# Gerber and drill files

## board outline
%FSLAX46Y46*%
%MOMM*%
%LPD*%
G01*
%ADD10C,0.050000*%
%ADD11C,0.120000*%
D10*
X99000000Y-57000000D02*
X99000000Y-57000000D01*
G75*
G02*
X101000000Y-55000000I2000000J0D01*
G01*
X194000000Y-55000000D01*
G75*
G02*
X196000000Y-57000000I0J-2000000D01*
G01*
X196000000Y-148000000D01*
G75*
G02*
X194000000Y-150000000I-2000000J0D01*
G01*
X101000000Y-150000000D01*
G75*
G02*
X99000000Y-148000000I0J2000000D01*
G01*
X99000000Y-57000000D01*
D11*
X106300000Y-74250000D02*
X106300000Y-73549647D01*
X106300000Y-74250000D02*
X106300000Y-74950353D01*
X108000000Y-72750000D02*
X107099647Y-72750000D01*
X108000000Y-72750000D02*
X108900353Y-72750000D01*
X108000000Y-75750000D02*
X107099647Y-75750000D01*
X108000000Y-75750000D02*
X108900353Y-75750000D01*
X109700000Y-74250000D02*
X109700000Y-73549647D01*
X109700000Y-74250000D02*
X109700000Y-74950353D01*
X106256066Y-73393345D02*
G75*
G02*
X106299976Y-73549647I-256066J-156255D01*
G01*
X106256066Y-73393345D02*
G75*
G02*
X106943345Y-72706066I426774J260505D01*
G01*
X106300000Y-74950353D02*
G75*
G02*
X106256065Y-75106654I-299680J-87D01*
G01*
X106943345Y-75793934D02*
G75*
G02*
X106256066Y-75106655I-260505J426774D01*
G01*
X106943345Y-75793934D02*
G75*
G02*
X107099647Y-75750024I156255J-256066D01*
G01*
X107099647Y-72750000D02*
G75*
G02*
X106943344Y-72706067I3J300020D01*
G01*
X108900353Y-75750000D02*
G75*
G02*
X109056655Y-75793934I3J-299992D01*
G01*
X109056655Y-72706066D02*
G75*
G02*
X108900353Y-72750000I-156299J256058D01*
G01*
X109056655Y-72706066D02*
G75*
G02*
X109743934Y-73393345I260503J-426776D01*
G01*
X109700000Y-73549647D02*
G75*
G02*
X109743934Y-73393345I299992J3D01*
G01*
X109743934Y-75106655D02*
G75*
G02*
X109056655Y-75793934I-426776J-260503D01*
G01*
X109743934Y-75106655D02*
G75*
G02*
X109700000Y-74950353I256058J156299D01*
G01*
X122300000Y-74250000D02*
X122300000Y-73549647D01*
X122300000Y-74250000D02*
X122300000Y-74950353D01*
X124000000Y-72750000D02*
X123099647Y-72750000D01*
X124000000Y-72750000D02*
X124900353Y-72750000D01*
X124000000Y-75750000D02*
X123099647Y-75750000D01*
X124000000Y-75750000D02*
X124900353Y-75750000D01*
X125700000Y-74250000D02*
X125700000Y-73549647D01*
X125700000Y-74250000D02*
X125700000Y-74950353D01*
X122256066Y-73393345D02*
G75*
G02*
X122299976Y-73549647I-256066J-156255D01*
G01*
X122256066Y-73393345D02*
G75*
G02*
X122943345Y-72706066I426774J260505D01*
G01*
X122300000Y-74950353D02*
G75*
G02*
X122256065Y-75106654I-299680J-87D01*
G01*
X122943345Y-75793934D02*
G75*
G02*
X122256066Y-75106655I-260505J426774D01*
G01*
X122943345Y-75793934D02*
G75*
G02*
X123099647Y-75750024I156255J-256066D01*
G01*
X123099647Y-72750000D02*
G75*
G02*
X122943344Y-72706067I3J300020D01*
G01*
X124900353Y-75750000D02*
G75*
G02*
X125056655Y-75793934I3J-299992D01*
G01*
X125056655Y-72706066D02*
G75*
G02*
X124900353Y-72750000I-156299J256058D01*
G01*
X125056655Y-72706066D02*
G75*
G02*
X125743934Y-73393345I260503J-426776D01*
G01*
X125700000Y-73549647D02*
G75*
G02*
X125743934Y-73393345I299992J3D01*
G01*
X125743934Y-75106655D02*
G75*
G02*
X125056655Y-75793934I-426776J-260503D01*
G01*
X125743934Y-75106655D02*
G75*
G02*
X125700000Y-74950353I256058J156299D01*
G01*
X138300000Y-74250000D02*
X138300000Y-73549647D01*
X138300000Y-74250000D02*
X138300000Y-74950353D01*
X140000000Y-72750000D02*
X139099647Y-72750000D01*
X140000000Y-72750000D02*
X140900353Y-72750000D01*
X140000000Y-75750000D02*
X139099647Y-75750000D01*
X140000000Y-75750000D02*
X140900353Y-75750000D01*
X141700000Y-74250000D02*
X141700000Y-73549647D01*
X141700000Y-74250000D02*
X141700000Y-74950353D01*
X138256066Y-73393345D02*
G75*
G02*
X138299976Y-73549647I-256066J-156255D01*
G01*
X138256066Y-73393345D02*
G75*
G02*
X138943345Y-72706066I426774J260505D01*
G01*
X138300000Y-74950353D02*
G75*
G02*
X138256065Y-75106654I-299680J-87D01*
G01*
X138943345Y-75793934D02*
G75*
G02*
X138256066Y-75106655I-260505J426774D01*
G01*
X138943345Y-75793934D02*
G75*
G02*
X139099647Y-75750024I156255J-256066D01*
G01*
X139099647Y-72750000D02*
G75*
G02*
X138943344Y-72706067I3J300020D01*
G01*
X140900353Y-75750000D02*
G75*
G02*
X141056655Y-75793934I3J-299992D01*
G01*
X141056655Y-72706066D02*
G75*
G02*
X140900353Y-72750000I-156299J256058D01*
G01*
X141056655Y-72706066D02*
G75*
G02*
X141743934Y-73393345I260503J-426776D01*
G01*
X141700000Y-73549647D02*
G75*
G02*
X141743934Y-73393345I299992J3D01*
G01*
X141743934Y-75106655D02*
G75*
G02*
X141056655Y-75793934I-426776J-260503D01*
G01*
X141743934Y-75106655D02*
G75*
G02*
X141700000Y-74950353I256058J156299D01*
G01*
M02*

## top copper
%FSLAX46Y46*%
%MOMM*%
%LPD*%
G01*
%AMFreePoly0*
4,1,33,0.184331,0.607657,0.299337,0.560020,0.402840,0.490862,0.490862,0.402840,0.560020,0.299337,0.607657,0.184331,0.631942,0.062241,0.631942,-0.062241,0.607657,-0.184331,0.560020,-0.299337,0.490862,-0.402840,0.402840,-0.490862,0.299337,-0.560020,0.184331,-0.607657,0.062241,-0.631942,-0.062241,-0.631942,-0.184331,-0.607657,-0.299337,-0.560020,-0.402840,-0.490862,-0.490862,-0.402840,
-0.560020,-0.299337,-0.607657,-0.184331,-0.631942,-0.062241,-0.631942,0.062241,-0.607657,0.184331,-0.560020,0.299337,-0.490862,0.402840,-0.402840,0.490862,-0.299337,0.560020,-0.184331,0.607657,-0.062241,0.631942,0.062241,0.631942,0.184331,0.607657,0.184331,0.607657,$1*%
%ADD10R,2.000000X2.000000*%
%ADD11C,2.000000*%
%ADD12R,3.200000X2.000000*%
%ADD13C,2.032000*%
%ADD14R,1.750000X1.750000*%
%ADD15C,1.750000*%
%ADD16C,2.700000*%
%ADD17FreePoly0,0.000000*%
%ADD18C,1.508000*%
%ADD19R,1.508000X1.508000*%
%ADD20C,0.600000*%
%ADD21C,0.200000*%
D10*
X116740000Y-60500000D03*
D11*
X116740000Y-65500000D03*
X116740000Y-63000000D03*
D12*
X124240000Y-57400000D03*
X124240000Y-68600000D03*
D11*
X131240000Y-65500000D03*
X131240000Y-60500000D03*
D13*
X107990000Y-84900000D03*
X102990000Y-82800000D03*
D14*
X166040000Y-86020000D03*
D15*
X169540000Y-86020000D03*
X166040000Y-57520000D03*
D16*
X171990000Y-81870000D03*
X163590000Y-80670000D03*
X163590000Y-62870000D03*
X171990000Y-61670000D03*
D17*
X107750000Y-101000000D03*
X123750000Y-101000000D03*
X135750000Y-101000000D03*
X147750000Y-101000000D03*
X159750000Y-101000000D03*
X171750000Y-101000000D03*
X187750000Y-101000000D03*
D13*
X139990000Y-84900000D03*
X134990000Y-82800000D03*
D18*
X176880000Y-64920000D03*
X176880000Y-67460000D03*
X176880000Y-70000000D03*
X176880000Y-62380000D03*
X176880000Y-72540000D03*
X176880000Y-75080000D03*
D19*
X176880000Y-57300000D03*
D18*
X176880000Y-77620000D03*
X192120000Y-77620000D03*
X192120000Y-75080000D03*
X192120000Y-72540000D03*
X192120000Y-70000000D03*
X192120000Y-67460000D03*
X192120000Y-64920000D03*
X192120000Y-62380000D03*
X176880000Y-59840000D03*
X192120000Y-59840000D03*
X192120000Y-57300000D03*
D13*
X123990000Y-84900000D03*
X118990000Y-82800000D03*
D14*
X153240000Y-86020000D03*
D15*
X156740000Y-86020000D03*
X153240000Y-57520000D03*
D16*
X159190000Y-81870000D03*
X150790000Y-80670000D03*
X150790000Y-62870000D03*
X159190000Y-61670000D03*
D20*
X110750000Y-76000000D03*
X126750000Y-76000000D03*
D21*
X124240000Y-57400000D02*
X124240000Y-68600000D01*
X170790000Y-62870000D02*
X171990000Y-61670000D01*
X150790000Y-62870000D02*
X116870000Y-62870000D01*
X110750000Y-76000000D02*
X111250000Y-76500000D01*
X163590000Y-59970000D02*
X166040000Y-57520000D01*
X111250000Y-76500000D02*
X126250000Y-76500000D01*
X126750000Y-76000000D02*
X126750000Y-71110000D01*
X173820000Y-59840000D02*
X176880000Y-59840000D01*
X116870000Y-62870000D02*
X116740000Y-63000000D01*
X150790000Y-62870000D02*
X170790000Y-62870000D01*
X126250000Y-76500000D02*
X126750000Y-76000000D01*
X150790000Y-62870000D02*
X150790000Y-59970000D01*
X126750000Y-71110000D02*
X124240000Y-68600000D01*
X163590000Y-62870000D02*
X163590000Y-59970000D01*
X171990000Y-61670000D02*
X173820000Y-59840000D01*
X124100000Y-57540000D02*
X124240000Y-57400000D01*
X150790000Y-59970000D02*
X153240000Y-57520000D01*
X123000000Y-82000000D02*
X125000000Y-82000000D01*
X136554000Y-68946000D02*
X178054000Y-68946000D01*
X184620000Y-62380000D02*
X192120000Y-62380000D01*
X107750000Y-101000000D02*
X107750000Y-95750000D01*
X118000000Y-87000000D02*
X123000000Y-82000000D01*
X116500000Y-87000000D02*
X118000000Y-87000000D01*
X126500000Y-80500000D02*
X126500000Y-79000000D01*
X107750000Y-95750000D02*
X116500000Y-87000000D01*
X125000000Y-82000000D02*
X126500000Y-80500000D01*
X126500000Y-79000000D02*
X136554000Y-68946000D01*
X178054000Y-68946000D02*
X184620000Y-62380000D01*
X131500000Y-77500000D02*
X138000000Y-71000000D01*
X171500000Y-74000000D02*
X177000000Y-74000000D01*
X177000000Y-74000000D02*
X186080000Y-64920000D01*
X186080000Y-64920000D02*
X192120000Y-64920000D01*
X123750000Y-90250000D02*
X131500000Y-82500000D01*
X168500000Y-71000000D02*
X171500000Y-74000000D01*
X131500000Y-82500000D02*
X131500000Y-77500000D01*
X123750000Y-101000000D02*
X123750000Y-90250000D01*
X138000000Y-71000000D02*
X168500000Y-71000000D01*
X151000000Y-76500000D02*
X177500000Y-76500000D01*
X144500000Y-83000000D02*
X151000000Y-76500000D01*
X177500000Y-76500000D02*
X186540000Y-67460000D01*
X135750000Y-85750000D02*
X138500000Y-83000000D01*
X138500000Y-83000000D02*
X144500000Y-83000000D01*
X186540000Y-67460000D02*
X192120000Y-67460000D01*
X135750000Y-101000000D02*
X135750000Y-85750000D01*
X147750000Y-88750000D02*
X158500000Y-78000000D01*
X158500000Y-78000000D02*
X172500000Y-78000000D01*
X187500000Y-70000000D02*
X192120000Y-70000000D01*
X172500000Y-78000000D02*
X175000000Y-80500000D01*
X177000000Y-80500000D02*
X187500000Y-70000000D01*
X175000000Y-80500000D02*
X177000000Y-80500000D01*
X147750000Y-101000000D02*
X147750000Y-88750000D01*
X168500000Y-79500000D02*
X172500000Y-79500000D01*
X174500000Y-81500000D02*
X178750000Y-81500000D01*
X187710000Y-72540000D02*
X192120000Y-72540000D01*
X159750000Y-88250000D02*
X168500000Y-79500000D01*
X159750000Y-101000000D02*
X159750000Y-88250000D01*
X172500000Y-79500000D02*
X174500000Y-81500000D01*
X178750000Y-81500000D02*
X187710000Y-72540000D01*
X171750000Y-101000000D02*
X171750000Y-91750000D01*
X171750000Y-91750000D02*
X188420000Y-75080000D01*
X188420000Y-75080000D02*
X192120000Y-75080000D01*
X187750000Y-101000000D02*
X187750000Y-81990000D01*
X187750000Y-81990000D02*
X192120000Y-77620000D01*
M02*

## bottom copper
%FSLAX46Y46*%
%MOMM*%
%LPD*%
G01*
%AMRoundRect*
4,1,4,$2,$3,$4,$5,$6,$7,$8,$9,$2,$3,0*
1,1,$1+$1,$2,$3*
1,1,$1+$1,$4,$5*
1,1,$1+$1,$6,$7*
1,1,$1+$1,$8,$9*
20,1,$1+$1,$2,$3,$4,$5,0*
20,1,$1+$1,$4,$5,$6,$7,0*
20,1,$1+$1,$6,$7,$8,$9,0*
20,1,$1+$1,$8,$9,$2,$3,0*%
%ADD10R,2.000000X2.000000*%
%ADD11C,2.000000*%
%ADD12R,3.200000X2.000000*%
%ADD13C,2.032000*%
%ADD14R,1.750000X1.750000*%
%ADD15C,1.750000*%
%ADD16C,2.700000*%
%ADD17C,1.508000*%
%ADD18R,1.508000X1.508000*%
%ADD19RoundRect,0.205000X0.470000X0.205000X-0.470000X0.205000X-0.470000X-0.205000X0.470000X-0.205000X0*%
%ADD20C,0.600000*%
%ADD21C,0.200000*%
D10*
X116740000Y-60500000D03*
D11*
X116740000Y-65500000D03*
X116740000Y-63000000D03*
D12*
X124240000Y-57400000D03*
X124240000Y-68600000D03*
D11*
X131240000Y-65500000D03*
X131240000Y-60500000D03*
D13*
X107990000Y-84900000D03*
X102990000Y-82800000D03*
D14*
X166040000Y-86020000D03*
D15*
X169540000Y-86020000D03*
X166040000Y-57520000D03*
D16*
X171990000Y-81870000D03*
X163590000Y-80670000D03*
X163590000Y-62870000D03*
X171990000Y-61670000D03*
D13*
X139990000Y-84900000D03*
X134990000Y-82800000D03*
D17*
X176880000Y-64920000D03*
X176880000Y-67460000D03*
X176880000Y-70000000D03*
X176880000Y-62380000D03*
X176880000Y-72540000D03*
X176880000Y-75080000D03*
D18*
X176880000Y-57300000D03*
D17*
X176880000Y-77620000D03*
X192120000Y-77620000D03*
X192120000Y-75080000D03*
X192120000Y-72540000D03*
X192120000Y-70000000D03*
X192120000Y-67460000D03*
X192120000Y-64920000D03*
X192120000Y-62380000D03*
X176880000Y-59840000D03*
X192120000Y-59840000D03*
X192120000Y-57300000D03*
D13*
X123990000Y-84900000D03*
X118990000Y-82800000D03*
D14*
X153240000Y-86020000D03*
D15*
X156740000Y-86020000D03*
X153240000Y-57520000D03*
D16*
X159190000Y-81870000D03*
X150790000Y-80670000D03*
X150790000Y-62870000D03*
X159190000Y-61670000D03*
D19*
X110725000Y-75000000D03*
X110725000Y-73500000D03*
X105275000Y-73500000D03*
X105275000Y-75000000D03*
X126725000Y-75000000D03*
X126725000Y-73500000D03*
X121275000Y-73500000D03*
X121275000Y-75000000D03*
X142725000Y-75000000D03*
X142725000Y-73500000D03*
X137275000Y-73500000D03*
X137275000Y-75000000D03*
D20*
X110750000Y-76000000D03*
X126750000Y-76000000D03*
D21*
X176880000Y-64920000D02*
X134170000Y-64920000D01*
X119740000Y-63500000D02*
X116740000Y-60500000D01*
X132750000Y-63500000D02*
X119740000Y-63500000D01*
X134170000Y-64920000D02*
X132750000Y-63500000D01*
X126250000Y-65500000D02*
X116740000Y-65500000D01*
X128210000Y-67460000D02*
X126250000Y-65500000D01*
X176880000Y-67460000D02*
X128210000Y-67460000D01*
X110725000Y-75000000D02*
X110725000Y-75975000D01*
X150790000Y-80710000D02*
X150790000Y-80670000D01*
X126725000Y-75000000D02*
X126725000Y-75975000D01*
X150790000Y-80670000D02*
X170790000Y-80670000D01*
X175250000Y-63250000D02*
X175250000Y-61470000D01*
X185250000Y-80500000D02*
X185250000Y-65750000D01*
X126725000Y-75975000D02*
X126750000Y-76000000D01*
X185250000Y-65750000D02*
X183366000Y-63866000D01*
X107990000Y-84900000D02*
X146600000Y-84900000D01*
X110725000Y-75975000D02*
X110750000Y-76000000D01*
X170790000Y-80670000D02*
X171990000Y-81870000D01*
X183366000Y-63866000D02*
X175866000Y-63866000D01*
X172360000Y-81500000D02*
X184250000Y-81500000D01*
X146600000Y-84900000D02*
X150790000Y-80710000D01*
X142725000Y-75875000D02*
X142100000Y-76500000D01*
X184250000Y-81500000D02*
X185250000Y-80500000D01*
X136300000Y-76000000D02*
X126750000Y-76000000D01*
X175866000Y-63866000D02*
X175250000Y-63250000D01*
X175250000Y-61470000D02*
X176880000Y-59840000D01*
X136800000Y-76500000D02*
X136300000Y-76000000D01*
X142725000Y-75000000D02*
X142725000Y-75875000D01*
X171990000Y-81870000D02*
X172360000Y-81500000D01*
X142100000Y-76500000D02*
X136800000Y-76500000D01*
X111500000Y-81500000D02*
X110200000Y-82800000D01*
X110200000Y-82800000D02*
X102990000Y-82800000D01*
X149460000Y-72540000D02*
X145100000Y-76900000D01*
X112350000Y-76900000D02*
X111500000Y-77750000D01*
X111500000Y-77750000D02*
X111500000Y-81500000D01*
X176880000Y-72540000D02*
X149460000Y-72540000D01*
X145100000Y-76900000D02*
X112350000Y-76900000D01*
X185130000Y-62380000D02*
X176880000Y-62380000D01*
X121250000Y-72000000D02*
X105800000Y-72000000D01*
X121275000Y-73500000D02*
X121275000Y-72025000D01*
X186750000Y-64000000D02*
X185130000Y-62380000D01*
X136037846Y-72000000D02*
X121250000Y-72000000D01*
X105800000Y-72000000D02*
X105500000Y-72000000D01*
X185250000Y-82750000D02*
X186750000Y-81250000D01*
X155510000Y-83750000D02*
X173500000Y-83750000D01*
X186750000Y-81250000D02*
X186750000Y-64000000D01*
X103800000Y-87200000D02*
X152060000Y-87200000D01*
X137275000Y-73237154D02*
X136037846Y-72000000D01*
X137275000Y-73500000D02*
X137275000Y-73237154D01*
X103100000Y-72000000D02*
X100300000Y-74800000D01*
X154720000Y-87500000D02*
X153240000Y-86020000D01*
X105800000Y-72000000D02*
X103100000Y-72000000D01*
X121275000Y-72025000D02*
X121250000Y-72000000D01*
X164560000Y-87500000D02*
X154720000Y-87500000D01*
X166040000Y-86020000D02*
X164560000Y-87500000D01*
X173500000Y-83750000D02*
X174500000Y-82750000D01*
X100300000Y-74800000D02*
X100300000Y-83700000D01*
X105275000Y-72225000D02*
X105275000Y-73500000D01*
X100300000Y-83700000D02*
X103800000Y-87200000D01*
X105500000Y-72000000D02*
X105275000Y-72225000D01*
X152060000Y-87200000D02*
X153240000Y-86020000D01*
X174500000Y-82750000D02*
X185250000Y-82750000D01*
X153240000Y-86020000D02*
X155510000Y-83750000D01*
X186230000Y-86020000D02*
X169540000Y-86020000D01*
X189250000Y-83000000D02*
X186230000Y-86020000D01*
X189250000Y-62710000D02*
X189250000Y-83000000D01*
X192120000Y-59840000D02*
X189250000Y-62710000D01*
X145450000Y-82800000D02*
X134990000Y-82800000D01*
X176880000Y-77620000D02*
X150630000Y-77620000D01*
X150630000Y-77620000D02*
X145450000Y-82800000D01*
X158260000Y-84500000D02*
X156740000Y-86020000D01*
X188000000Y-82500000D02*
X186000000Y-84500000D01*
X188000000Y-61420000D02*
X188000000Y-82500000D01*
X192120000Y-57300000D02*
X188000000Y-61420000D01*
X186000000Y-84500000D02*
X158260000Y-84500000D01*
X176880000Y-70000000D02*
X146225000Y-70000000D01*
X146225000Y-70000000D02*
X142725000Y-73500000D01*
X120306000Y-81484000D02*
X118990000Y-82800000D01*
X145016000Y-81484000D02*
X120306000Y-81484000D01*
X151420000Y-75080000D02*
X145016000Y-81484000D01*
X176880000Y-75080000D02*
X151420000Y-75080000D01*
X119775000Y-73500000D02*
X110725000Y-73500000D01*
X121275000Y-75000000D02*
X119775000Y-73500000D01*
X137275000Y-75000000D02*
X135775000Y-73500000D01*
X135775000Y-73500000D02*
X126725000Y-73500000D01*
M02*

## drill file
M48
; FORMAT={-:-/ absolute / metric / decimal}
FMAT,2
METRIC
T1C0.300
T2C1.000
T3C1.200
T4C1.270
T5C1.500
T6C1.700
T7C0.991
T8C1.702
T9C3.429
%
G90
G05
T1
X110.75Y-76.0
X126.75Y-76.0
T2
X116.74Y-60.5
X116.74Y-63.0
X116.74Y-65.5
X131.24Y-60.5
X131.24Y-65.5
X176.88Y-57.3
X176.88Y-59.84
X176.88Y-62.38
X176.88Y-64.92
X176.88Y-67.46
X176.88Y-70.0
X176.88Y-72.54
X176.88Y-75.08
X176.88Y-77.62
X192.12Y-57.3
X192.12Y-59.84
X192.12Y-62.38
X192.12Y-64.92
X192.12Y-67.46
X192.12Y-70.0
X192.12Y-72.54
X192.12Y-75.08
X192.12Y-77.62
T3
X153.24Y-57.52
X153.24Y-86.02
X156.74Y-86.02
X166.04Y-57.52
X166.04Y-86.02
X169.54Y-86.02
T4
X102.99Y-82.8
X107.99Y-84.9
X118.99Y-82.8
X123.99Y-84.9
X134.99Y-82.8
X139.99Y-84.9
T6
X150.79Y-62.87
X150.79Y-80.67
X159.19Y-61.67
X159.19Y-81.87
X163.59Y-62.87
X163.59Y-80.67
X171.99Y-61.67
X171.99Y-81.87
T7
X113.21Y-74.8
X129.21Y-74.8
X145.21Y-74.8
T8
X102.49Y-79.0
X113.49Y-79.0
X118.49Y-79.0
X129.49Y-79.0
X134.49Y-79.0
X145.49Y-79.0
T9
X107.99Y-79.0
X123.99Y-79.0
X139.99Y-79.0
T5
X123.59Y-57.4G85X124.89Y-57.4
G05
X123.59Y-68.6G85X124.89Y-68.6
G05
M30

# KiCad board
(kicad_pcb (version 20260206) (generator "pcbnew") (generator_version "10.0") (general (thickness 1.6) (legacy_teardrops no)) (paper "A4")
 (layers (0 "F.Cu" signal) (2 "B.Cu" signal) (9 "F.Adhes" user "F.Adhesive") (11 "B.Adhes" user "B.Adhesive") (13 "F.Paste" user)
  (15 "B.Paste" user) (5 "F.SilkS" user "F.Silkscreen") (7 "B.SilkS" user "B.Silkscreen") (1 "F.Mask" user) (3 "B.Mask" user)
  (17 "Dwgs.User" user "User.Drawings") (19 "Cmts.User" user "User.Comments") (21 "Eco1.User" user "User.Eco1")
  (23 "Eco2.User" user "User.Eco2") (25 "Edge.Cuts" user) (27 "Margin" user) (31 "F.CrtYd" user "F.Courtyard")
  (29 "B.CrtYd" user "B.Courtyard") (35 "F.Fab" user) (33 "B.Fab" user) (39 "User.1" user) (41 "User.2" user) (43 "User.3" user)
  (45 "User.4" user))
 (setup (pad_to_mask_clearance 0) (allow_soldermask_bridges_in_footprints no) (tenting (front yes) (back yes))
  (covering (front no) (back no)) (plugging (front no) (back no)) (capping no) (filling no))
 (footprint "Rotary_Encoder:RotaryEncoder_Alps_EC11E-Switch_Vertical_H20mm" (layer "F.Cu") (at 116.74 60.5)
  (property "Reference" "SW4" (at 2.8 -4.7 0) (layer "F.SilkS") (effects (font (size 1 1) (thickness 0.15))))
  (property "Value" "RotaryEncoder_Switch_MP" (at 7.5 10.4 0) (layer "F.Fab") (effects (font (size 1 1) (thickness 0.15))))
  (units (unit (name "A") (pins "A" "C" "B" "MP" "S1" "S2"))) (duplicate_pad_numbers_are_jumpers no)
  (pad "A" thru_hole rect (at 0 0) (size 2 2) (drill 1) (layers "*.Cu" "*.Mask") (remove_unused_layers no) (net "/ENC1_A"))
  (pad "B" thru_hole circle (at 0 5) (size 2 2) (drill 1) (layers "*.Cu" "*.Mask") (remove_unused_layers no) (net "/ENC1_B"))
  (pad "C" thru_hole circle (at 0 2.5) (size 2 2) (drill 1) (layers "*.Cu" "*.Mask") (remove_unused_layers no) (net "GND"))
  (pad "MP" thru_hole rect (at 7.5 -3.1) (size 3.2 2) (drill oval 2.8 1.5) (layers "*.Cu" "*.Mask") (remove_unused_layers no) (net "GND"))
  (pad "MP" thru_hole rect (at 7.5 8.1) (size 3.2 2) (drill oval 2.8 1.5) (layers "*.Cu" "*.Mask") (remove_unused_layers no) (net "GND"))
  (pad "S1" thru_hole circle (at 14.5 5) (size 2 2) (drill 1) (layers "*.Cu" "*.Mask") (remove_unused_layers no)
   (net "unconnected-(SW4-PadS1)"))
  (pad "S2" thru_hole circle (at 14.5 0) (size 2 2) (drill 1) (layers "*.Cu" "*.Mask") (remove_unused_layers no)
   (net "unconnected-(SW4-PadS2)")))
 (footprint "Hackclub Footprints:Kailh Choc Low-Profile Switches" (layer "F.Cu") (at 107.99 79)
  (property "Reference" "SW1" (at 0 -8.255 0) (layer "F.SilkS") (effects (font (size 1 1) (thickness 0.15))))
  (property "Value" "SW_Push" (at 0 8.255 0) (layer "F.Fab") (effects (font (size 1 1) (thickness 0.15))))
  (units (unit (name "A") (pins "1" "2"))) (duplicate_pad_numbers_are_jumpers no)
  (pad "" np_thru_hole circle (at -5.5 0) (size 1.7018 1.7018) (drill 1.7018) (layers "*.Cu" "*.Mask"))
  (pad "" np_thru_hole circle (at 0 0) (size 3.429 3.429) (drill 3.429) (layers "*.Cu" "*.Mask"))
  (pad "" np_thru_hole circle (at 5.22 -4.2) (size 0.9906 0.9906) (drill 0.9906) (layers "*.Cu" "*.Mask"))
  (pad "" np_thru_hole circle (at 5.5 0) (size 1.7018 1.7018) (drill 1.7018) (layers "*.Cu" "*.Mask"))
  (pad "1" thru_hole circle (at 0 5.9) (size 2.032 2.032) (drill 1.27) (layers "*.Cu" "*.Mask") (remove_unused_layers no) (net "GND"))
  (pad "2" thru_hole circle (at -5 3.8) (size 2.032 2.032) (drill 1.27) (layers "*.Cu" "*.Mask") (remove_unused_layers no) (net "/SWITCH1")))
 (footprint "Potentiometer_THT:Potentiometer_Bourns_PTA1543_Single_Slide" (layer "F.Cu") (at 166.04 86.02 90)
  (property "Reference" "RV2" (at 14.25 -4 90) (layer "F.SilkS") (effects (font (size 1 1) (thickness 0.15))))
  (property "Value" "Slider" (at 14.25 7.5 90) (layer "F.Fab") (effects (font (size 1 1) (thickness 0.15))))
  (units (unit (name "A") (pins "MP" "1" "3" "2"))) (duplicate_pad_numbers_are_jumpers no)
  (pad "1" thru_hole rect (at 0 0 90) (size 1.75 1.75) (drill 1.2) (layers "*.Cu" "*.Mask") (remove_unused_layers no) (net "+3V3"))
  (pad "2" thru_hole circle (at 0 3.5 90) (size 1.75 1.75) (drill 1.2) (layers "*.Cu" "*.Mask") (remove_unused_layers no) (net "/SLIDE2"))
  (pad "3" thru_hole circle (at 28.5 0 90) (size 1.75 1.75) (drill 1.2) (layers "*.Cu" "*.Mask") (remove_unused_layers no) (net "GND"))
  (pad "MP" thru_hole circle (at 4.15 5.95 90) (size 2.7 2.7) (drill 1.7) (layers "*.Cu" "*.Mask") (remove_unused_layers no) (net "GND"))
  (pad "MP" thru_hole circle (at 5.35 -2.45 90) (size 2.7 2.7) (drill 1.7) (layers "*.Cu" "*.Mask") (remove_unused_layers no) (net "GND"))
  (pad "MP" thru_hole circle (at 23.15 -2.45 90) (size 2.7 2.7) (drill 1.7) (layers "*.Cu" "*.Mask") (remove_unused_layers no) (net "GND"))
  (pad "MP" thru_hole circle (at 24.35 5.95 90) (size 2.7 2.7) (drill 1.7) (layers "*.Cu" "*.Mask") (remove_unused_layers no) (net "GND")))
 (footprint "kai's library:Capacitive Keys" (layer "F.Cu") (at 147.75 81)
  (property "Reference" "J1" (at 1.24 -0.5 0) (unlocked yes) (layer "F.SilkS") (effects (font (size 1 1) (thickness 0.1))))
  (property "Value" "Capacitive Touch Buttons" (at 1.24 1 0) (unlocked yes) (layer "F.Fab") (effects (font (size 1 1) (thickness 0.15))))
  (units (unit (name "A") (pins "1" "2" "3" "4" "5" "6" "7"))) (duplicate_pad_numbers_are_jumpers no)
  (pad "1" smd custom (at -40 20) (size 1.27 1.27) (layers "F.Cu" "F.Mask") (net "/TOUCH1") (thermal_bridge_angle 90)
   (options (clearance outline) (anchor circle)) (primitives))
  (pad "2" smd custom (at -24 20) (size 1.27 1.27) (layers "F.Cu" "F.Mask") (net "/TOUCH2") (thermal_bridge_angle 90)
   (options (clearance outline) (anchor circle)) (primitives))
  (pad "3" smd custom (at -12 20) (size 1.27 1.27) (layers "F.Cu" "F.Mask") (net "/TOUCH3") (thermal_bridge_angle 90)
   (options (clearance outline) (anchor circle)) (primitives))
  (pad "4" smd custom (at 0 20) (size 1.27 1.27) (layers "F.Cu" "F.Mask") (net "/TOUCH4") (thermal_bridge_angle 90)
   (options (clearance outline) (anchor circle)) (primitives))
  (pad "5" smd custom (at 12 20) (size 1.27 1.27) (layers "F.Cu" "F.Mask") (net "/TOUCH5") (thermal_bridge_angle 90)
   (options (clearance outline) (anchor circle)) (primitives))
  (pad "6" smd custom (at 24 20) (size 1.27 1.27) (layers "F.Cu" "F.Mask") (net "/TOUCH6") (thermal_bridge_angle 90)
   (options (clearance outline) (anchor circle)) (primitives))
  (pad "7" smd custom (at 40 20) (size 1.27 1.27) (layers "F.Cu" "F.Mask") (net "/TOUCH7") (thermal_bridge_angle 90)
   (options (clearance outline) (anchor circle)) (primitives)))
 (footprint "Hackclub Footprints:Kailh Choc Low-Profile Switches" (layer "F.Cu") (at 139.99 79)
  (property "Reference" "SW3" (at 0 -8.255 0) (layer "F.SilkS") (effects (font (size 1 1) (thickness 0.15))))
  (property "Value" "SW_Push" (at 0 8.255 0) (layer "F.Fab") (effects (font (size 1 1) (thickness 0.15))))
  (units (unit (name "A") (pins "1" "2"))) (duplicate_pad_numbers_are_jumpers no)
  (pad "" np_thru_hole circle (at -5.5 0) (size 1.7018 1.7018) (drill 1.7018) (layers "*.Cu" "*.Mask"))
  (pad "" np_thru_hole circle (at 0 0) (size 3.429 3.429) (drill 3.429) (layers "*.Cu" "*.Mask"))
  (pad "" np_thru_hole circle (at 5.22 -4.2) (size 0.9906 0.9906) (drill 0.9906) (layers "*.Cu" "*.Mask"))
  (pad "" np_thru_hole circle (at 5.5 0) (size 1.7018 1.7018) (drill 1.7018) (layers "*.Cu" "*.Mask"))
  (pad "1" thru_hole circle (at 0 5.9) (size 2.032 2.032) (drill 1.27) (layers "*.Cu" "*.Mask") (remove_unused_layers no) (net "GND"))
  (pad "2" thru_hole circle (at -5 3.8) (size 2.032 2.032) (drill 1.27) (layers "*.Cu" "*.Mask") (remove_unused_layers no) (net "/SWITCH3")))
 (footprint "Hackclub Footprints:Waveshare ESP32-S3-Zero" (layer "F.Cu") (at 184.5 67.46)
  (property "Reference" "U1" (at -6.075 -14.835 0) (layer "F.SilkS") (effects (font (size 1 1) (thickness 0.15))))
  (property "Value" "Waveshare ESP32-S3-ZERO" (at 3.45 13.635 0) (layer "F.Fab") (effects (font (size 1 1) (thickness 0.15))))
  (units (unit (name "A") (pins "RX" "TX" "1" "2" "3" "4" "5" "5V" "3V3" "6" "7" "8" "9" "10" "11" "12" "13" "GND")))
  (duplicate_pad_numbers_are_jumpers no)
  (pad "1" thru_hole circle (at -7.62 -2.54) (size 1.508 1.508) (drill 1) (layers "*.Cu" "*.Mask") (remove_unused_layers no) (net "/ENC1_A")
   (solder_mask_margin 0.102))
  (pad "2" thru_hole circle (at -7.62 0) (size 1.508 1.508) (drill 1) (layers "*.Cu" "*.Mask") (remove_unused_layers no) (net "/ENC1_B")
   (solder_mask_margin 0.102))
  (pad "3" thru_hole circle (at -7.62 2.54) (size 1.508 1.508) (drill 1) (layers "*.Cu" "*.Mask") (remove_unused_layers no) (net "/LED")
   (solder_mask_margin 0.102))
  (pad "3V3" thru_hole circle (at -7.62 -5.08) (size 1.508 1.508) (drill 1) (layers "*.Cu" "*.Mask") (remove_unused_layers no) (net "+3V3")
   (solder_mask_margin 0.102))
  (pad "4" thru_hole circle (at -7.62 5.08) (size 1.508 1.508) (drill 1) (layers "*.Cu" "*.Mask") (remove_unused_layers no) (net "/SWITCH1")
   (solder_mask_margin 0.102))
  (pad "5" thru_hole circle (at -7.62 7.62) (size 1.508 1.508) (drill 1) (layers "*.Cu" "*.Mask") (remove_unused_layers no) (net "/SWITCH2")
   (solder_mask_margin 0.102))
  (pad "5V" thru_hole rect (at -7.62 -10.16) (size 1.508 1.508) (drill 1) (layers "*.Cu" "*.Mask") (remove_unused_layers no) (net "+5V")
   (solder_mask_margin 0.102))
  (pad "6" thru_hole circle (at -7.62 10.16) (size 1.508 1.508) (drill 1) (layers "*.Cu" "*.Mask") (remove_unused_layers no)
   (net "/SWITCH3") (solder_mask_margin 0.102))
  (pad "7" thru_hole circle (at 7.62 10.16) (size 1.508 1.508) (drill 1) (layers "*.Cu" "*.Mask") (remove_unused_layers no) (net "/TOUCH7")
   (solder_mask_margin 0.102))
  (pad "8" thru_hole circle (at 7.62 7.62) (size 1.508 1.508) (drill 1) (layers "*.Cu" "*.Mask") (remove_unused_layers no) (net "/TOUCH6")
   (solder_mask_margin 0.102))
  (pad "9" thru_hole circle (at 7.62 5.08) (size 1.508 1.508) (drill 1) (layers "*.Cu" "*.Mask") (remove_unused_layers no) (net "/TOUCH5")
   (solder_mask_margin 0.102))
  (pad "10" thru_hole circle (at 7.62 2.54) (size 1.508 1.508) (drill 1) (layers "*.Cu" "*.Mask") (remove_unused_layers no) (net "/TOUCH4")
   (solder_mask_margin 0.102))
  (pad "11" thru_hole circle (at 7.62 0) (size 1.508 1.508) (drill 1) (layers "*.Cu" "*.Mask") (remove_unused_layers no) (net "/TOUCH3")
   (solder_mask_margin 0.102))
  (pad "12" thru_hole circle (at 7.62 -2.54) (size 1.508 1.508) (drill 1) (layers "*.Cu" "*.Mask") (remove_unused_layers no) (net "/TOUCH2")
   (solder_mask_margin 0.102))
  (pad "13" thru_hole circle (at 7.62 -5.08) (size 1.508 1.508) (drill 1) (layers "*.Cu" "*.Mask") (remove_unused_layers no) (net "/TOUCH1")
   (solder_mask_margin 0.102))
  (pad "GND" thru_hole circle (at -7.62 -7.62) (size 1.508 1.508) (drill 1) (layers "*.Cu" "*.Mask") (remove_unused_layers no) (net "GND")
   (solder_mask_margin 0.102))
  (pad "RX" thru_hole circle (at 7.62 -7.62) (size 1.508 1.508) (drill 1) (layers "*.Cu" "*.Mask") (remove_unused_layers no) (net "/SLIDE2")
   (solder_mask_margin 0.102))
  (pad "TX" thru_hole circle (at 7.62 -10.16) (size 1.508 1.508) (drill 1) (layers "*.Cu" "*.Mask") (remove_unused_layers no)
   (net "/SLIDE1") (solder_mask_margin 0.102)))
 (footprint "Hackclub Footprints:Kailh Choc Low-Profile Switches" (layer "F.Cu") (at 123.99 79)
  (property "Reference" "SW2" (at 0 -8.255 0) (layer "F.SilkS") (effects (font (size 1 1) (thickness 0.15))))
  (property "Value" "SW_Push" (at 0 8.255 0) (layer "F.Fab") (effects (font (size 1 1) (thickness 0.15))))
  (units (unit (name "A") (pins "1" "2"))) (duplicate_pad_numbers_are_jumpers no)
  (pad "" np_thru_hole circle (at -5.5 0) (size 1.7018 1.7018) (drill 1.7018) (layers "*.Cu" "*.Mask"))
  (pad "" np_thru_hole circle (at 0 0) (size 3.429 3.429) (drill 3.429) (layers "*.Cu" "*.Mask"))
  (pad "" np_thru_hole circle (at 5.22 -4.2) (size 0.9906 0.9906) (drill 0.9906) (layers "*.Cu" "*.Mask"))
  (pad "" np_thru_hole circle (at 5.5 0) (size 1.7018 1.7018) (drill 1.7018) (layers "*.Cu" "*.Mask"))
  (pad "1" thru_hole circle (at 0 5.9) (size 2.032 2.032) (drill 1.27) (layers "*.Cu" "*.Mask") (remove_unused_layers no) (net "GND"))
  (pad "2" thru_hole circle (at -5 3.8) (size 2.032 2.032) (drill 1.27) (layers "*.Cu" "*.Mask") (remove_unused_layers no) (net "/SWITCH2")))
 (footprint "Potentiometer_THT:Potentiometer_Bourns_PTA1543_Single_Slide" (layer "F.Cu") (at 153.24 86.02 90)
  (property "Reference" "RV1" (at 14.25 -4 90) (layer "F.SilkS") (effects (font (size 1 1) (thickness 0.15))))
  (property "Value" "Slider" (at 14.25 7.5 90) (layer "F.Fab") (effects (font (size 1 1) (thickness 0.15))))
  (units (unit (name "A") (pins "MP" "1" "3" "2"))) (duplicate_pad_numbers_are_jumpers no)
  (pad "1" thru_hole rect (at 0 0 90) (size 1.75 1.75) (drill 1.2) (layers "*.Cu" "*.Mask") (remove_unused_layers no) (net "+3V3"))
  (pad "2" thru_hole circle (at 0 3.5 90) (size 1.75 1.75) (drill 1.2) (layers "*.Cu" "*.Mask") (remove_unused_layers no) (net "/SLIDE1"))
  (pad "3" thru_hole circle (at 28.5 0 90) (size 1.75 1.75) (drill 1.2) (layers "*.Cu" "*.Mask") (remove_unused_layers no) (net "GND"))
  (pad "MP" thru_hole circle (at 4.15 5.95 90) (size 2.7 2.7) (drill 1.7) (layers "*.Cu" "*.Mask") (remove_unused_layers no) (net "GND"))
  (pad "MP" thru_hole circle (at 5.35 -2.45 90) (size 2.7 2.7) (drill 1.7) (layers "*.Cu" "*.Mask") (remove_unused_layers no) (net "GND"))
  (pad "MP" thru_hole circle (at 23.15 -2.45 90) (size 2.7 2.7) (drill 1.7) (layers "*.Cu" "*.Mask") (remove_unused_layers no) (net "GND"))
  (pad "MP" thru_hole circle (at 24.35 5.95 90) (size 2.7 2.7) (drill 1.7) (layers "*.Cu" "*.Mask") (remove_unused_layers no) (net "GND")))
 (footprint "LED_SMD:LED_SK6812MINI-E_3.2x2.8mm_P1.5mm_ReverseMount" (layer "B.Cu") (at 108 74.25 180)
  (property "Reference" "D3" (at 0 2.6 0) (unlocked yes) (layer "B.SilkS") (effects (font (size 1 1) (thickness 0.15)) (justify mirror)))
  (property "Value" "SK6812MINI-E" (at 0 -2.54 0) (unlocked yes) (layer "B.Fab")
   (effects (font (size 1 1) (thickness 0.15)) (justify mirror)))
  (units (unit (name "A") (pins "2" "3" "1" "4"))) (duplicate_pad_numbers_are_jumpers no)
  (fp_line (start 1.7 0) (end 1.7 0.700353) (stroke (width 0.12) (type solid)) (layer "Edge.Cuts"))
  (fp_line (start 1.7 0) (end 1.7 -0.700353) (stroke (width 0.12) (type solid)) (layer "Edge.Cuts"))
  (fp_line (start 0 1.5) (end 0.900353 1.5) (stroke (width 0.12) (type solid)) (layer "Edge.Cuts"))
  (fp_line (start 0 1.5) (end -0.900353 1.5) (stroke (width 0.12) (type solid)) (layer "Edge.Cuts"))
  (fp_line (start 0 -1.5) (end 0.900353 -1.5) (stroke (width 0.12) (type solid)) (layer "Edge.Cuts"))
  (fp_line (start 0 -1.5) (end -0.900353 -1.5) (stroke (width 0.12) (type solid)) (layer "Edge.Cuts"))
  (fp_line (start -1.7 0) (end -1.7 0.700353) (stroke (width 0.12) (type solid)) (layer "Edge.Cuts"))
  (fp_line (start -1.7 0) (end -1.7 -0.700353) (stroke (width 0.12) (type solid)) (layer "Edge.Cuts"))
  (fp_arc (start 1.743934 0.856655) (mid 1.711191 0.781533) (end 1.7 0.700353) (stroke (width 0.12) (type solid)) (layer "Edge.Cuts"))
  (fp_arc (start 1.743934 0.856655) (mid 1.670713 1.470713) (end 1.056655 1.543934) (stroke (width 0.12) (type solid)) (layer "Edge.Cuts"))
  (fp_arc (start 1.7 -0.700353) (mid 1.711181 -0.781538) (end 1.743934 -0.856655) (stroke (width 0.12) (type solid)) (layer "Edge.Cuts"))
  (fp_arc (start 1.056655 -1.543934) (mid 1.670711 -1.470711) (end 1.743934 -0.856655) (stroke (width 0.12) (type solid))
   (layer "Edge.Cuts"))
  (fp_arc (start 1.056655 -1.543934) (mid 0.981533 -1.511191) (end 0.900353 -1.5) (stroke (width 0.12) (type solid)) (layer "Edge.Cuts"))
  (fp_arc (start 0.900353 1.5) (mid 0.981532 1.511193) (end 1.056655 1.543934) (stroke (width 0.12) (type solid)) (layer "Edge.Cuts"))
  (fp_arc (start -0.900353 -1.5) (mid -0.981533 -1.511192) (end -1.056655 -1.543934) (stroke (width 0.12) (type solid)) (layer "Edge.Cuts"))
  (fp_arc (start -1.056655 1.543934) (mid -0.981533 1.511192) (end -0.900353 1.5) (stroke (width 0.12) (type solid)) (layer "Edge.Cuts"))
  (fp_arc (start -1.056655 1.543934) (mid -1.670711 1.470711) (end -1.743934 0.856655) (stroke (width 0.12) (type solid))
   (layer "Edge.Cuts"))
  (fp_arc (start -1.7 0.700353) (mid -1.711192 0.781533) (end -1.743934 0.856655) (stroke (width 0.12) (type solid)) (layer "Edge.Cuts"))
  (fp_arc (start -1.743934 -0.856655) (mid -1.670711 -1.470711) (end -1.056655 -1.543934) (stroke (width 0.12) (type solid))
   (layer "Edge.Cuts"))
  (fp_arc (start -1.743934 -0.856655) (mid -1.711192 -0.781533) (end -1.7 -0.700353) (stroke (width 0.12) (type solid)) (layer "Edge.Cuts"))
  (pad "1" smd roundrect (at -2.725 -0.75 180) (size 1.35 0.82) (layers "B.Cu" "B.Mask" "B.Paste") (roundrect_rratio 0.25) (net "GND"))
  (pad "2" smd roundrect (at -2.725 0.75 180) (size 1.35 0.82) (layers "B.Cu" "B.Mask" "B.Paste") (roundrect_rratio 0.25)
   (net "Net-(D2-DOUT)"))
  (pad "3" smd roundrect (at 2.725 0.75 180) (size 1.35 0.82) (layers "B.Cu" "B.Mask" "B.Paste") (roundrect_rratio 0.25) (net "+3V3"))
  (pad "4" smd roundrect (at 2.725 -0.75 180) (size 1.35 0.82) (layers "B.Cu" "B.Mask" "B.Paste") (roundrect_rratio 0.25)
   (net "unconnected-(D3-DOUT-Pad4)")))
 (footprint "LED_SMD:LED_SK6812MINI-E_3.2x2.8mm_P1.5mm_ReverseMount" (layer "B.Cu") (at 124 74.25 180)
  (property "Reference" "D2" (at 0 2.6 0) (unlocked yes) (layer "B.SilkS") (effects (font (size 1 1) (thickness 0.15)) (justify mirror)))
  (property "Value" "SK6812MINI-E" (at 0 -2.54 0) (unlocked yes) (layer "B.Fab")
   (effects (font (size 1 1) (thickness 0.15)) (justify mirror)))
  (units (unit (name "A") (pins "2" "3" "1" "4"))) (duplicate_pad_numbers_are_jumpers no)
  (fp_line (start 1.7 0) (end 1.7 0.700353) (stroke (width 0.12) (type solid)) (layer "Edge.Cuts"))
  (fp_line (start 1.7 0) (end 1.7 -0.700353) (stroke (width 0.12) (type solid)) (layer "Edge.Cuts"))
  (fp_line (start 0 1.5) (end 0.900353 1.5) (stroke (width 0.12) (type solid)) (layer "Edge.Cuts"))
  (fp_line (start 0 1.5) (end -0.900353 1.5) (stroke (width 0.12) (type solid)) (layer "Edge.Cuts"))
  (fp_line (start 0 -1.5) (end 0.900353 -1.5) (stroke (width 0.12) (type solid)) (layer "Edge.Cuts"))
  (fp_line (start 0 -1.5) (end -0.900353 -1.5) (stroke (width 0.12) (type solid)) (layer "Edge.Cuts"))
  (fp_line (start -1.7 0) (end -1.7 0.700353) (stroke (width 0.12) (type solid)) (layer "Edge.Cuts"))
  (fp_line (start -1.7 0) (end -1.7 -0.700353) (stroke (width 0.12) (type solid)) (layer "Edge.Cuts"))
  (fp_arc (start 1.743934 0.856655) (mid 1.711191 0.781533) (end 1.7 0.700353) (stroke (width 0.12) (type solid)) (layer "Edge.Cuts"))
  (fp_arc (start 1.743934 0.856655) (mid 1.670713 1.470713) (end 1.056655 1.543934) (stroke (width 0.12) (type solid)) (layer "Edge.Cuts"))
  (fp_arc (start 1.7 -0.700353) (mid 1.711181 -0.781538) (end 1.743934 -0.856655) (stroke (width 0.12) (type solid)) (layer "Edge.Cuts"))
  (fp_arc (start 1.056655 -1.543934) (mid 1.670711 -1.470711) (end 1.743934 -0.856655) (stroke (width 0.12) (type solid))
   (layer "Edge.Cuts"))
  (fp_arc (start 1.056655 -1.543934) (mid 0.981533 -1.511191) (end 0.900353 -1.5) (stroke (width 0.12) (type solid)) (layer "Edge.Cuts"))
  (fp_arc (start 0.900353 1.5) (mid 0.981532 1.511193) (end 1.056655 1.543934) (stroke (width 0.12) (type solid)) (layer "Edge.Cuts"))
  (fp_arc (start -0.900353 -1.5) (mid -0.981533 -1.511192) (end -1.056655 -1.543934) (stroke (width 0.12) (type solid)) (layer "Edge.Cuts"))
  (fp_arc (start -1.056655 1.543934) (mid -0.981533 1.511192) (end -0.900353 1.5) (stroke (width 0.12) (type solid)) (layer "Edge.Cuts"))
  (fp_arc (start -1.056655 1.543934) (mid -1.670711 1.470711) (end -1.743934 0.856655) (stroke (width 0.12) (type solid))
   (layer "Edge.Cuts"))
  (fp_arc (start -1.7 0.700353) (mid -1.711192 0.781533) (end -1.743934 0.856655) (stroke (width 0.12) (type solid)) (layer "Edge.Cuts"))
  (fp_arc (start -1.743934 -0.856655) (mid -1.670711 -1.470711) (end -1.056655 -1.543934) (stroke (width 0.12) (type solid))
   (layer "Edge.Cuts"))
  (fp_arc (start -1.743934 -0.856655) (mid -1.711192 -0.781533) (end -1.7 -0.700353) (stroke (width 0.12) (type solid)) (layer "Edge.Cuts"))
  (pad "1" smd roundrect (at -2.725 -0.75 180) (size 1.35 0.82) (layers "B.Cu" "B.Mask" "B.Paste") (roundrect_rratio 0.25) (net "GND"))
  (pad "2" smd roundrect (at -2.725 0.75 180) (size 1.35 0.82) (layers "B.Cu" "B.Mask" "B.Paste") (roundrect_rratio 0.25)
   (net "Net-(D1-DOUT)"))
  (pad "3" smd roundrect (at 2.725 0.75 180) (size 1.35 0.82) (layers "B.Cu" "B.Mask" "B.Paste") (roundrect_rratio 0.25) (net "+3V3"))
  (pad "4" smd roundrect (at 2.725 -0.75 180) (size 1.35 0.82) (layers "B.Cu" "B.Mask" "B.Paste") (roundrect_rratio 0.25)
   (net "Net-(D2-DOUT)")))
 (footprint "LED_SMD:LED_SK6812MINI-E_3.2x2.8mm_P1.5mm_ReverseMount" (layer "B.Cu") (at 140 74.25 180)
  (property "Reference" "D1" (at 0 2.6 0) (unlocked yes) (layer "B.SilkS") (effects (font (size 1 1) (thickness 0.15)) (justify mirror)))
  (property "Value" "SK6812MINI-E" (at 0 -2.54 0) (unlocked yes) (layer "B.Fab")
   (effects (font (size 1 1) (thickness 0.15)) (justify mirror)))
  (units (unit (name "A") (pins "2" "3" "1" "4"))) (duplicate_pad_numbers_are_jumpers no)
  (fp_line (start 1.7 0) (end 1.7 0.700353) (stroke (width 0.12) (type solid)) (layer "Edge.Cuts"))
  (fp_line (start 1.7 0) (end 1.7 -0.700353) (stroke (width 0.12) (type solid)) (layer "Edge.Cuts"))
  (fp_line (start 0 1.5) (end 0.900353 1.5) (stroke (width 0.12) (type solid)) (layer "Edge.Cuts"))
  (fp_line (start 0 1.5) (end -0.900353 1.5) (stroke (width 0.12) (type solid)) (layer "Edge.Cuts"))
  (fp_line (start 0 -1.5) (end 0.900353 -1.5) (stroke (width 0.12) (type solid)) (layer "Edge.Cuts"))
  (fp_line (start 0 -1.5) (end -0.900353 -1.5) (stroke (width 0.12) (type solid)) (layer "Edge.Cuts"))
  (fp_line (start -1.7 0) (end -1.7 0.700353) (stroke (width 0.12) (type solid)) (layer "Edge.Cuts"))
  (fp_line (start -1.7 0) (end -1.7 -0.700353) (stroke (width 0.12) (type solid)) (layer "Edge.Cuts"))
  (fp_arc (start 1.743934 0.856655) (mid 1.711191 0.781533) (end 1.7 0.700353) (stroke (width 0.12) (type solid)) (layer "Edge.Cuts"))
  (fp_arc (start 1.743934 0.856655) (mid 1.670713 1.470713) (end 1.056655 1.543934) (stroke (width 0.12) (type solid)) (layer "Edge.Cuts"))
  (fp_arc (start 1.7 -0.700353) (mid 1.711181 -0.781538) (end 1.743934 -0.856655) (stroke (width 0.12) (type solid)) (layer "Edge.Cuts"))
  (fp_arc (start 1.056655 -1.543934) (mid 1.670711 -1.470711) (end 1.743934 -0.856655) (stroke (width 0.12) (type solid))
   (layer "Edge.Cuts"))
  (fp_arc (start 1.056655 -1.543934) (mid 0.981533 -1.511191) (end 0.900353 -1.5) (stroke (width 0.12) (type solid)) (layer "Edge.Cuts"))
  (fp_arc (start 0.900353 1.5) (mid 0.981532 1.511193) (end 1.056655 1.543934) (stroke (width 0.12) (type solid)) (layer "Edge.Cuts"))
  (fp_arc (start -0.900353 -1.5) (mid -0.981533 -1.511192) (end -1.056655 -1.543934) (stroke (width 0.12) (type solid)) (layer "Edge.Cuts"))
  (fp_arc (start -1.056655 1.543934) (mid -0.981533 1.511192) (end -0.900353 1.5) (stroke (width 0.12) (type solid)) (layer "Edge.Cuts"))
  (fp_arc (start -1.056655 1.543934) (mid -1.670711 1.470711) (end -1.743934 0.856655) (stroke (width 0.12) (type solid))
   (layer "Edge.Cuts"))
  (fp_arc (start -1.7 0.700353) (mid -1.711192 0.781533) (end -1.743934 0.856655) (stroke (width 0.12) (type solid)) (layer "Edge.Cuts"))
  (fp_arc (start -1.743934 -0.856655) (mid -1.670711 -1.470711) (end -1.056655 -1.543934) (stroke (width 0.12) (type solid))
   (layer "Edge.Cuts"))
  (fp_arc (start -1.743934 -0.856655) (mid -1.711192 -0.781533) (end -1.7 -0.700353) (stroke (width 0.12) (type solid)) (layer "Edge.Cuts"))
  (pad "1" smd roundrect (at -2.725 -0.75 180) (size 1.35 0.82) (layers "B.Cu" "B.Mask" "B.Paste") (roundrect_rratio 0.25) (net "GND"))
  (pad "2" smd roundrect (at -2.725 0.75 180) (size 1.35 0.82) (layers "B.Cu" "B.Mask" "B.Paste") (roundrect_rratio 0.25) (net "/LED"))
  (pad "3" smd roundrect (at 2.725 0.75 180) (size 1.35 0.82) (layers "B.Cu" "B.Mask" "B.Paste") (roundrect_rratio 0.25) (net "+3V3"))
  (pad "4" smd roundrect (at 2.725 -0.75 180) (size 1.35 0.82) (layers "B.Cu" "B.Mask" "B.Paste") (roundrect_rratio 0.25)
   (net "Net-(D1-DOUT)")))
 (gr_rect (start 99 55) (end 196 150) (radius 2) (stroke (width 0.05) (type solid)) (fill no) (layer "Edge.Cuts"))
 (segment (start 176.88 64.92) (end 134.17 64.92) (width 0.2) (layer "B.Cu") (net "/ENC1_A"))
 (segment (start 119.74 63.5) (end 116.74 60.5) (width 0.2) (layer "B.Cu") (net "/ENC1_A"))
 (segment (start 132.75 63.5) (end 119.74 63.5) (width 0.2) (layer "B.Cu") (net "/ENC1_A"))
 (segment (start 134.17 64.92) (end 132.75 63.5) (width 0.2) (layer "B.Cu") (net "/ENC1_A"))
 (segment (start 126.25 65.5) (end 116.74 65.5) (width 0.2) (layer "B.Cu") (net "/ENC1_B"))
 (segment (start 128.21 67.46) (end 126.25 65.5) (width 0.2) (layer "B.Cu") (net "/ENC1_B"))
 (segment (start 176.88 67.46) (end 128.21 67.46) (width 0.2) (layer "B.Cu") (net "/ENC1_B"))
 (segment (start 124.24 57.4) (end 124.24 68.6) (width 0.2) (layer "F.Cu") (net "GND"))
 (segment (start 170.79 62.87) (end 171.99 61.67) (width 0.2) (layer "F.Cu") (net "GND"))
 (segment (start 150.79 62.87) (end 116.87 62.87) (width 0.2) (layer "F.Cu") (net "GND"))
 (segment (start 110.75 76) (end 111.25 76.5) (width 0.2) (layer "F.Cu") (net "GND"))
 (segment (start 163.59 59.97) (end 166.04 57.52) (width 0.2) (layer "F.Cu") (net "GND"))
 (segment (start 111.25 76.5) (end 126.25 76.5) (width 0.2) (layer "F.Cu") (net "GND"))
 (segment (start 126.75 76) (end 126.75 71.11) (width 0.2) (layer "F.Cu") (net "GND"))
 (segment (start 173.82 59.84) (end 176.88 59.84) (width 0.2) (layer "F.Cu") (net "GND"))
 (segment (start 116.87 62.87) (end 116.74 63) (width 0.2) (layer "F.Cu") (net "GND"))
 (segment (start 150.79 62.87) (end 170.79 62.87) (width 0.2) (layer "F.Cu") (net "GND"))
 (segment (start 126.25 76.5) (end 126.75 76) (width 0.2) (layer "F.Cu") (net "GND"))
 (segment (start 150.79 62.87) (end 150.79 59.97) (width 0.2) (layer "F.Cu") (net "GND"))
 (segment (start 126.75 71.11) (end 124.24 68.6) (width 0.2) (layer "F.Cu") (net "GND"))
 (segment (start 163.59 62.87) (end 163.59 59.97) (width 0.2) (layer "F.Cu") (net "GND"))
 (segment (start 171.99 61.67) (end 173.82 59.84) (width 0.2) (layer "F.Cu") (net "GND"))
 (segment (start 124.1 57.54) (end 124.24 57.4) (width 0.2) (layer "F.Cu") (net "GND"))
 (segment (start 150.79 59.97) (end 153.24 57.52) (width 0.2) (layer "F.Cu") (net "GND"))
 (via (at 110.75 76) (size 0.6) (drill 0.3) (layers "F.Cu" "B.Cu") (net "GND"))
 (via (at 126.75 76) (size 0.6) (drill 0.3) (layers "F.Cu" "B.Cu") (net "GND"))
 (segment (start 110.725 75) (end 110.725 75.975) (width 0.2) (layer "B.Cu") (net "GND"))
 (segment (start 150.79 80.71) (end 150.79 80.67) (width 0.2) (layer "B.Cu") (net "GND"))
 (segment (start 126.725 75) (end 126.725 75.975) (width 0.2) (layer "B.Cu") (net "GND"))
 (segment (start 150.79 80.67) (end 170.79 80.67) (width 0.2) (layer "B.Cu") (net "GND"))
 (segment (start 175.25 63.25) (end 175.25 61.47) (width 0.2) (layer "B.Cu") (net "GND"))
 (segment (start 185.25 80.5) (end 185.25 65.75) (width 0.2) (layer "B.Cu") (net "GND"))
 (segment (start 126.725 75.975) (end 126.75 76) (width 0.2) (layer "B.Cu") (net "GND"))
 (segment (start 185.25 65.75) (end 183.366 63.866) (width 0.2) (layer "B.Cu") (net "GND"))
 (segment (start 107.99 84.9) (end 146.6 84.9) (width 0.2) (layer "B.Cu") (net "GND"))
 (segment (start 110.725 75.975) (end 110.75 76) (width 0.2) (layer "B.Cu") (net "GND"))
 (segment (start 170.79 80.67) (end 171.99 81.87) (width 0.2) (layer "B.Cu") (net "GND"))
 (segment (start 183.366 63.866) (end 175.866 63.866) (width 0.2) (layer "B.Cu") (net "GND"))
 (segment (start 172.36 81.5) (end 184.25 81.5) (width 0.2) (layer "B.Cu") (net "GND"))
 (segment (start 146.6 84.9) (end 150.79 80.71) (width 0.2) (layer "B.Cu") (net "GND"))
 (segment (start 142.725 75.875) (end 142.1 76.5) (width 0.2) (layer "B.Cu") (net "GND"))
 (segment (start 184.25 81.5) (end 185.25 80.5) (width 0.2) (layer "B.Cu") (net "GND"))
 (segment (start 136.3 76) (end 126.75 76) (width 0.2) (layer "B.Cu") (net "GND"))
 (segment (start 175.866 63.866) (end 175.25 63.25) (width 0.2) (layer "B.Cu") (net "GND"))
 (segment (start 175.25 61.47) (end 176.88 59.84) (width 0.2) (layer "B.Cu") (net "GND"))
 (segment (start 136.8 76.5) (end 136.3 76) (width 0.2) (layer "B.Cu") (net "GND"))
 (segment (start 142.725 75) (end 142.725 75.875) (width 0.2) (layer "B.Cu") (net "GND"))
 (segment (start 171.99 81.87) (end 172.36 81.5) (width 0.2) (layer "B.Cu") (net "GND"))
 (segment (start 142.1 76.5) (end 136.8 76.5) (width 0.2) (layer "B.Cu") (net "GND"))
 (segment (start 111.5 81.5) (end 110.2 82.8) (width 0.2) (layer "B.Cu") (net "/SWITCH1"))
 (segment (start 110.2 82.8) (end 102.99 82.8) (width 0.2) (layer "B.Cu") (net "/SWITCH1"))
 (segment (start 149.46 72.54) (end 145.1 76.9) (width 0.2) (layer "B.Cu") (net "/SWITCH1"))
 (segment (start 112.35 76.9) (end 111.5 77.75) (width 0.2) (layer "B.Cu") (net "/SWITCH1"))
 (segment (start 111.5 77.75) (end 111.5 81.5) (width 0.2) (layer "B.Cu") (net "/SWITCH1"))
 (segment (start 176.88 72.54) (end 149.46 72.54) (width 0.2) (layer "B.Cu") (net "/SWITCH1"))
 (segment (start 145.1 76.9) (end 112.35 76.9) (width 0.2) (layer "B.Cu") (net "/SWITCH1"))
 (segment (start 185.13 62.38) (end 176.88 62.38) (width 0.2) (layer "B.Cu") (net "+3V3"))
 (segment (start 121.25 72) (end 105.8 72) (width 0.2) (layer "B.Cu") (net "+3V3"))
 (segment (start 121.275 73.5) (end 121.275 72.025) (width 0.2) (layer "B.Cu") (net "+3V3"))
 (segment (start 186.75 64) (end 185.13 62.38) (width 0.2) (layer "B.Cu") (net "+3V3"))
 (segment (start 136.037846 72) (end 121.25 72) (width 0.2) (layer "B.Cu") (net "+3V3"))
 (segment (start 105.8 72) (end 105.5 72) (width 0.2) (layer "B.Cu") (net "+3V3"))
 (segment (start 185.25 82.75) (end 186.75 81.25) (width 0.2) (layer "B.Cu") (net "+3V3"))
 (segment (start 155.51 83.75) (end 173.5 83.75) (width 0.2) (layer "B.Cu") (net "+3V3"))
 (segment (start 186.75 81.25) (end 186.75 64) (width 0.2) (layer "B.Cu") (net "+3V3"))
 (segment (start 103.8 87.2) (end 152.06 87.2) (width 0.2) (layer "B.Cu") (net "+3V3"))
 (segment (start 137.275 73.237154) (end 136.037846 72) (width 0.2) (layer "B.Cu") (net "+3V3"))
 (segment (start 137.275 73.5) (end 137.275 73.237154) (width 0.2) (layer "B.Cu") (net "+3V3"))
 (segment (start 103.1 72) (end 100.3 74.8) (width 0.2) (layer "B.Cu") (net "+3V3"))
 (segment (start 154.72 87.5) (end 153.24 86.02) (width 0.2) (layer "B.Cu") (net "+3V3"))
 (segment (start 105.8 72) (end 103.1 72) (width 0.2) (layer "B.Cu") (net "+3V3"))
 (segment (start 121.275 72.025) (end 121.25 72) (width 0.2) (layer "B.Cu") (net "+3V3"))
 (segment (start 164.56 87.5) (end 154.72 87.5) (width 0.2) (layer "B.Cu") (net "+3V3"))
 (segment (start 166.04 86.02) (end 164.56 87.5) (width 0.2) (layer "B.Cu") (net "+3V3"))
 (segment (start 173.5 83.75) (end 174.5 82.75) (width 0.2) (layer "B.Cu") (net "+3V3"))
 (segment (start 100.3 74.8) (end 100.3 83.7) (width 0.2) (layer "B.Cu") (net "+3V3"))
 (segment (start 105.275 72.225) (end 105.275 73.5) (width 0.2) (layer "B.Cu") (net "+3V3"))
 (segment (start 100.3 83.7) (end 103.8 87.2) (width 0.2) (layer "B.Cu") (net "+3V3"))
 (segment (start 105.5 72) (end 105.275 72.225) (width 0.2) (layer "B.Cu") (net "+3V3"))
 (segment (start 152.06 87.2) (end 153.24 86.02) (width 0.2) (layer "B.Cu") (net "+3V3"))
 (segment (start 174.5 82.75) (end 185.25 82.75) (width 0.2) (layer "B.Cu") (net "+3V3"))
 (segment (start 153.24 86.02) (end 155.51 83.75) (width 0.2) (layer "B.Cu") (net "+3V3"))
 (segment (start 186.23 86.02) (end 169.54 86.02) (width 0.2) (layer "B.Cu") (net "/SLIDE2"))
 (segment (start 189.25 83) (end 186.23 86.02) (width 0.2) (layer "B.Cu") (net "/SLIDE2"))
 (segment (start 189.25 62.71) (end 189.25 83) (width 0.2) (layer "B.Cu") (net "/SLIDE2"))
 (segment (start 192.12 59.84) (end 189.25 62.71) (width 0.2) (layer "B.Cu") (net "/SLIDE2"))
 (segment (start 123 82) (end 125 82) (width 0.2) (layer "F.Cu") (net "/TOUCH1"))
 (segment (start 136.554 68.946) (end 178.054 68.946) (width 0.2) (layer "F.Cu") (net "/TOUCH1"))
 (segment (start 184.62 62.38) (end 192.12 62.38) (width 0.2) (layer "F.Cu") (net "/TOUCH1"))
 (segment (start 107.75 101) (end 107.75 95.75) (width 0.2) (layer "F.Cu") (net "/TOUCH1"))
 (segment (start 118 87) (end 123 82) (width 0.2) (layer "F.Cu") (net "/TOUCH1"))
 (segment (start 116.5 87) (end 118 87) (width 0.2) (layer "F.Cu") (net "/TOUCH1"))
 (segment (start 126.5 80.5) (end 126.5 79) (width 0.2) (layer "F.Cu") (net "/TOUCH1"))
 (segment (start 107.75 95.75) (end 116.5 87) (width 0.2) (layer "F.Cu") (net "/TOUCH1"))
 (segment (start 125 82) (end 126.5 80.5) (width 0.2) (layer "F.Cu") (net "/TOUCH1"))
 (segment (start 126.5 79) (end 136.554 68.946) (width 0.2) (layer "F.Cu") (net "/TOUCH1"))
 (segment (start 178.054 68.946) (end 184.62 62.38) (width 0.2) (layer "F.Cu") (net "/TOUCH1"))
 (segment (start 131.5 77.5) (end 138 71) (width 0.2) (layer "F.Cu") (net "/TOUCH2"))
 (segment (start 171.5 74) (end 177 74) (width 0.2) (layer "F.Cu") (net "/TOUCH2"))
 (segment (start 177 74) (end 186.08 64.92) (width 0.2) (layer "F.Cu") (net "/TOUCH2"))
 (segment (start 186.08 64.92) (end 192.12 64.92) (width 0.2) (layer "F.Cu") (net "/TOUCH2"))
 (segment (start 123.75 90.25) (end 131.5 82.5) (width 0.2) (layer "F.Cu") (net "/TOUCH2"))
 (segment (start 168.5 71) (end 171.5 74) (width 0.2) (layer "F.Cu") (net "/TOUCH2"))
 (segment (start 131.5 82.5) (end 131.5 77.5) (width 0.2) (layer "F.Cu") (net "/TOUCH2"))
 (segment (start 123.75 101) (end 123.75 90.25) (width 0.2) (layer "F.Cu") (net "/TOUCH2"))
 (segment (start 138 71) (end 168.5 71) (width 0.2) (layer "F.Cu") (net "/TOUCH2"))
 (segment (start 151 76.5) (end 177.5 76.5) (width 0.2) (layer "F.Cu") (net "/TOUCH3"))
 (segment (start 144.5 83) (end 151 76.5) (width 0.2) (layer "F.Cu") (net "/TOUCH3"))
 (segment (start 177.5 76.5) (end 186.54 67.46) (width 0.2) (layer "F.Cu") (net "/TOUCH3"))
 (segment (start 135.75 85.75) (end 138.5 83) (width 0.2) (layer "F.Cu") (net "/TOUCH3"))
 (segment (start 138.5 83) (end 144.5 83) (width 0.2) (layer "F.Cu") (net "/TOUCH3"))
 (segment (start 186.54 67.46) (end 192.12 67.46) (width 0.2) (layer "F.Cu") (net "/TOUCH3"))
 (segment (start 135.75 101) (end 135.75 85.75) (width 0.2) (layer "F.Cu") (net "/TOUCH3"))
 (segment (start 147.75 88.75) (end 158.5 78) (width 0.2) (layer "F.Cu") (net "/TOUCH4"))
 (segment (start 158.5 78) (end 172.5 78) (width 0.2) (layer "F.Cu") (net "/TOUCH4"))
 (segment (start 187.5 70) (end 192.12 70) (width 0.2) (layer "F.Cu") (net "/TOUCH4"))
 (segment (start 172.5 78) (end 175 80.5) (width 0.2) (layer "F.Cu") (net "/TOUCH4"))
 (segment (start 177 80.5) (end 187.5 70) (width 0.2) (layer "F.Cu") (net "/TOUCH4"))
 (segment (start 175 80.5) (end 177 80.5) (width 0.2) (layer "F.Cu") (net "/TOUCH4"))
 (segment (start 147.75 101) (end 147.75 88.75) (width 0.2) (layer "F.Cu") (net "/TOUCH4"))
 (segment (start 168.5 79.5) (end 172.5 79.5) (width 0.2) (layer "F.Cu") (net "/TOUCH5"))
 (segment (start 174.5 81.5) (end 178.75 81.5) (width 0.2) (layer "F.Cu") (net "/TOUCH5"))
 (segment (start 187.71 72.54) (end 192.12 72.54) (width 0.2) (layer "F.Cu") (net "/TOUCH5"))
 (segment (start 159.75 88.25) (end 168.5 79.5) (width 0.2) (layer "F.Cu") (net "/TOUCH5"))
 (segment (start 159.75 101) (end 159.75 88.25) (width 0.2) (layer "F.Cu") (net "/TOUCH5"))
 (segment (start 172.5 79.5) (end 174.5 81.5) (width 0.2) (layer "F.Cu") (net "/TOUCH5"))
 (segment (start 178.75 81.5) (end 187.71 72.54) (width 0.2) (layer "F.Cu") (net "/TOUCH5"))
 (segment (start 171.75 101) (end 171.75 91.75) (width 0.2) (layer "F.Cu") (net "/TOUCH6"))
 (segment (start 171.75 91.75) (end 188.42 75.08) (width 0.2) (layer "F.Cu") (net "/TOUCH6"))
 (segment (start 188.42 75.08) (end 192.12 75.08) (width 0.2) (layer "F.Cu") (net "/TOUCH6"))
 (segment (start 187.75 101) (end 187.75 81.99) (width 0.2) (layer "F.Cu") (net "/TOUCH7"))
 (segment (start 187.75 81.99) (end 192.12 77.62) (width 0.2) (layer "F.Cu") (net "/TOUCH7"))
 (segment (start 145.45 82.8) (end 134.99 82.8) (width 0.2) (layer "B.Cu") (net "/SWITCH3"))
 (segment (start 176.88 77.62) (end 150.63 77.62) (width 0.2) (layer "B.Cu") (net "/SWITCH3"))
 (segment (start 150.63 77.62) (end 145.45 82.8) (width 0.2) (layer "B.Cu") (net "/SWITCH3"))
 (segment (start 158.26 84.5) (end 156.74 86.02) (width 0.2) (layer "B.Cu") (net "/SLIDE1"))
 (segment (start 188 82.5) (end 186 84.5) (width 0.2) (layer "B.Cu") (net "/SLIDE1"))
 (segment (start 188 61.42) (end 188 82.5) (width 0.2) (layer "B.Cu") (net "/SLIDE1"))
 (segment (start 192.12 57.3) (end 188 61.42) (width 0.2) (layer "B.Cu") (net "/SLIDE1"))
 (segment (start 186 84.5) (end 158.26 84.5) (width 0.2) (layer "B.Cu") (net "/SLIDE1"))
 (segment (start 176.88 70) (end 146.225 70) (width 0.2) (layer "B.Cu") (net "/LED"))
 (segment (start 146.225 70) (end 142.725 73.5) (width 0.2) (layer "B.Cu") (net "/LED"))
 (segment (start 120.306 81.484) (end 118.99 82.8) (width 0.2) (layer "B.Cu") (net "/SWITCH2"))
 (segment (start 145.016 81.484) (end 120.306 81.484) (width 0.2) (layer "B.Cu") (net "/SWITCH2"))
 (segment (start 151.42 75.08) (end 145.016 81.484) (width 0.2) (layer "B.Cu") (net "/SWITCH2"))
 (segment (start 176.88 75.08) (end 151.42 75.08) (width 0.2) (layer "B.Cu") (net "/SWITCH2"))
 (segment (start 119.775 73.5) (end 110.725 73.5) (width 0.2) (layer "B.Cu") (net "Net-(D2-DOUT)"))
 (segment (start 121.275 75) (end 119.775 73.5) (width 0.2) (layer "B.Cu") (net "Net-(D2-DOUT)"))
 (segment (start 137.275 75) (end 135.775 73.5) (width 0.2) (layer "B.Cu") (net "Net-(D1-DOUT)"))
 (segment (start 135.775 73.5) (end 126.725 73.5) (width 0.2) (layer "B.Cu") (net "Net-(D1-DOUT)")))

